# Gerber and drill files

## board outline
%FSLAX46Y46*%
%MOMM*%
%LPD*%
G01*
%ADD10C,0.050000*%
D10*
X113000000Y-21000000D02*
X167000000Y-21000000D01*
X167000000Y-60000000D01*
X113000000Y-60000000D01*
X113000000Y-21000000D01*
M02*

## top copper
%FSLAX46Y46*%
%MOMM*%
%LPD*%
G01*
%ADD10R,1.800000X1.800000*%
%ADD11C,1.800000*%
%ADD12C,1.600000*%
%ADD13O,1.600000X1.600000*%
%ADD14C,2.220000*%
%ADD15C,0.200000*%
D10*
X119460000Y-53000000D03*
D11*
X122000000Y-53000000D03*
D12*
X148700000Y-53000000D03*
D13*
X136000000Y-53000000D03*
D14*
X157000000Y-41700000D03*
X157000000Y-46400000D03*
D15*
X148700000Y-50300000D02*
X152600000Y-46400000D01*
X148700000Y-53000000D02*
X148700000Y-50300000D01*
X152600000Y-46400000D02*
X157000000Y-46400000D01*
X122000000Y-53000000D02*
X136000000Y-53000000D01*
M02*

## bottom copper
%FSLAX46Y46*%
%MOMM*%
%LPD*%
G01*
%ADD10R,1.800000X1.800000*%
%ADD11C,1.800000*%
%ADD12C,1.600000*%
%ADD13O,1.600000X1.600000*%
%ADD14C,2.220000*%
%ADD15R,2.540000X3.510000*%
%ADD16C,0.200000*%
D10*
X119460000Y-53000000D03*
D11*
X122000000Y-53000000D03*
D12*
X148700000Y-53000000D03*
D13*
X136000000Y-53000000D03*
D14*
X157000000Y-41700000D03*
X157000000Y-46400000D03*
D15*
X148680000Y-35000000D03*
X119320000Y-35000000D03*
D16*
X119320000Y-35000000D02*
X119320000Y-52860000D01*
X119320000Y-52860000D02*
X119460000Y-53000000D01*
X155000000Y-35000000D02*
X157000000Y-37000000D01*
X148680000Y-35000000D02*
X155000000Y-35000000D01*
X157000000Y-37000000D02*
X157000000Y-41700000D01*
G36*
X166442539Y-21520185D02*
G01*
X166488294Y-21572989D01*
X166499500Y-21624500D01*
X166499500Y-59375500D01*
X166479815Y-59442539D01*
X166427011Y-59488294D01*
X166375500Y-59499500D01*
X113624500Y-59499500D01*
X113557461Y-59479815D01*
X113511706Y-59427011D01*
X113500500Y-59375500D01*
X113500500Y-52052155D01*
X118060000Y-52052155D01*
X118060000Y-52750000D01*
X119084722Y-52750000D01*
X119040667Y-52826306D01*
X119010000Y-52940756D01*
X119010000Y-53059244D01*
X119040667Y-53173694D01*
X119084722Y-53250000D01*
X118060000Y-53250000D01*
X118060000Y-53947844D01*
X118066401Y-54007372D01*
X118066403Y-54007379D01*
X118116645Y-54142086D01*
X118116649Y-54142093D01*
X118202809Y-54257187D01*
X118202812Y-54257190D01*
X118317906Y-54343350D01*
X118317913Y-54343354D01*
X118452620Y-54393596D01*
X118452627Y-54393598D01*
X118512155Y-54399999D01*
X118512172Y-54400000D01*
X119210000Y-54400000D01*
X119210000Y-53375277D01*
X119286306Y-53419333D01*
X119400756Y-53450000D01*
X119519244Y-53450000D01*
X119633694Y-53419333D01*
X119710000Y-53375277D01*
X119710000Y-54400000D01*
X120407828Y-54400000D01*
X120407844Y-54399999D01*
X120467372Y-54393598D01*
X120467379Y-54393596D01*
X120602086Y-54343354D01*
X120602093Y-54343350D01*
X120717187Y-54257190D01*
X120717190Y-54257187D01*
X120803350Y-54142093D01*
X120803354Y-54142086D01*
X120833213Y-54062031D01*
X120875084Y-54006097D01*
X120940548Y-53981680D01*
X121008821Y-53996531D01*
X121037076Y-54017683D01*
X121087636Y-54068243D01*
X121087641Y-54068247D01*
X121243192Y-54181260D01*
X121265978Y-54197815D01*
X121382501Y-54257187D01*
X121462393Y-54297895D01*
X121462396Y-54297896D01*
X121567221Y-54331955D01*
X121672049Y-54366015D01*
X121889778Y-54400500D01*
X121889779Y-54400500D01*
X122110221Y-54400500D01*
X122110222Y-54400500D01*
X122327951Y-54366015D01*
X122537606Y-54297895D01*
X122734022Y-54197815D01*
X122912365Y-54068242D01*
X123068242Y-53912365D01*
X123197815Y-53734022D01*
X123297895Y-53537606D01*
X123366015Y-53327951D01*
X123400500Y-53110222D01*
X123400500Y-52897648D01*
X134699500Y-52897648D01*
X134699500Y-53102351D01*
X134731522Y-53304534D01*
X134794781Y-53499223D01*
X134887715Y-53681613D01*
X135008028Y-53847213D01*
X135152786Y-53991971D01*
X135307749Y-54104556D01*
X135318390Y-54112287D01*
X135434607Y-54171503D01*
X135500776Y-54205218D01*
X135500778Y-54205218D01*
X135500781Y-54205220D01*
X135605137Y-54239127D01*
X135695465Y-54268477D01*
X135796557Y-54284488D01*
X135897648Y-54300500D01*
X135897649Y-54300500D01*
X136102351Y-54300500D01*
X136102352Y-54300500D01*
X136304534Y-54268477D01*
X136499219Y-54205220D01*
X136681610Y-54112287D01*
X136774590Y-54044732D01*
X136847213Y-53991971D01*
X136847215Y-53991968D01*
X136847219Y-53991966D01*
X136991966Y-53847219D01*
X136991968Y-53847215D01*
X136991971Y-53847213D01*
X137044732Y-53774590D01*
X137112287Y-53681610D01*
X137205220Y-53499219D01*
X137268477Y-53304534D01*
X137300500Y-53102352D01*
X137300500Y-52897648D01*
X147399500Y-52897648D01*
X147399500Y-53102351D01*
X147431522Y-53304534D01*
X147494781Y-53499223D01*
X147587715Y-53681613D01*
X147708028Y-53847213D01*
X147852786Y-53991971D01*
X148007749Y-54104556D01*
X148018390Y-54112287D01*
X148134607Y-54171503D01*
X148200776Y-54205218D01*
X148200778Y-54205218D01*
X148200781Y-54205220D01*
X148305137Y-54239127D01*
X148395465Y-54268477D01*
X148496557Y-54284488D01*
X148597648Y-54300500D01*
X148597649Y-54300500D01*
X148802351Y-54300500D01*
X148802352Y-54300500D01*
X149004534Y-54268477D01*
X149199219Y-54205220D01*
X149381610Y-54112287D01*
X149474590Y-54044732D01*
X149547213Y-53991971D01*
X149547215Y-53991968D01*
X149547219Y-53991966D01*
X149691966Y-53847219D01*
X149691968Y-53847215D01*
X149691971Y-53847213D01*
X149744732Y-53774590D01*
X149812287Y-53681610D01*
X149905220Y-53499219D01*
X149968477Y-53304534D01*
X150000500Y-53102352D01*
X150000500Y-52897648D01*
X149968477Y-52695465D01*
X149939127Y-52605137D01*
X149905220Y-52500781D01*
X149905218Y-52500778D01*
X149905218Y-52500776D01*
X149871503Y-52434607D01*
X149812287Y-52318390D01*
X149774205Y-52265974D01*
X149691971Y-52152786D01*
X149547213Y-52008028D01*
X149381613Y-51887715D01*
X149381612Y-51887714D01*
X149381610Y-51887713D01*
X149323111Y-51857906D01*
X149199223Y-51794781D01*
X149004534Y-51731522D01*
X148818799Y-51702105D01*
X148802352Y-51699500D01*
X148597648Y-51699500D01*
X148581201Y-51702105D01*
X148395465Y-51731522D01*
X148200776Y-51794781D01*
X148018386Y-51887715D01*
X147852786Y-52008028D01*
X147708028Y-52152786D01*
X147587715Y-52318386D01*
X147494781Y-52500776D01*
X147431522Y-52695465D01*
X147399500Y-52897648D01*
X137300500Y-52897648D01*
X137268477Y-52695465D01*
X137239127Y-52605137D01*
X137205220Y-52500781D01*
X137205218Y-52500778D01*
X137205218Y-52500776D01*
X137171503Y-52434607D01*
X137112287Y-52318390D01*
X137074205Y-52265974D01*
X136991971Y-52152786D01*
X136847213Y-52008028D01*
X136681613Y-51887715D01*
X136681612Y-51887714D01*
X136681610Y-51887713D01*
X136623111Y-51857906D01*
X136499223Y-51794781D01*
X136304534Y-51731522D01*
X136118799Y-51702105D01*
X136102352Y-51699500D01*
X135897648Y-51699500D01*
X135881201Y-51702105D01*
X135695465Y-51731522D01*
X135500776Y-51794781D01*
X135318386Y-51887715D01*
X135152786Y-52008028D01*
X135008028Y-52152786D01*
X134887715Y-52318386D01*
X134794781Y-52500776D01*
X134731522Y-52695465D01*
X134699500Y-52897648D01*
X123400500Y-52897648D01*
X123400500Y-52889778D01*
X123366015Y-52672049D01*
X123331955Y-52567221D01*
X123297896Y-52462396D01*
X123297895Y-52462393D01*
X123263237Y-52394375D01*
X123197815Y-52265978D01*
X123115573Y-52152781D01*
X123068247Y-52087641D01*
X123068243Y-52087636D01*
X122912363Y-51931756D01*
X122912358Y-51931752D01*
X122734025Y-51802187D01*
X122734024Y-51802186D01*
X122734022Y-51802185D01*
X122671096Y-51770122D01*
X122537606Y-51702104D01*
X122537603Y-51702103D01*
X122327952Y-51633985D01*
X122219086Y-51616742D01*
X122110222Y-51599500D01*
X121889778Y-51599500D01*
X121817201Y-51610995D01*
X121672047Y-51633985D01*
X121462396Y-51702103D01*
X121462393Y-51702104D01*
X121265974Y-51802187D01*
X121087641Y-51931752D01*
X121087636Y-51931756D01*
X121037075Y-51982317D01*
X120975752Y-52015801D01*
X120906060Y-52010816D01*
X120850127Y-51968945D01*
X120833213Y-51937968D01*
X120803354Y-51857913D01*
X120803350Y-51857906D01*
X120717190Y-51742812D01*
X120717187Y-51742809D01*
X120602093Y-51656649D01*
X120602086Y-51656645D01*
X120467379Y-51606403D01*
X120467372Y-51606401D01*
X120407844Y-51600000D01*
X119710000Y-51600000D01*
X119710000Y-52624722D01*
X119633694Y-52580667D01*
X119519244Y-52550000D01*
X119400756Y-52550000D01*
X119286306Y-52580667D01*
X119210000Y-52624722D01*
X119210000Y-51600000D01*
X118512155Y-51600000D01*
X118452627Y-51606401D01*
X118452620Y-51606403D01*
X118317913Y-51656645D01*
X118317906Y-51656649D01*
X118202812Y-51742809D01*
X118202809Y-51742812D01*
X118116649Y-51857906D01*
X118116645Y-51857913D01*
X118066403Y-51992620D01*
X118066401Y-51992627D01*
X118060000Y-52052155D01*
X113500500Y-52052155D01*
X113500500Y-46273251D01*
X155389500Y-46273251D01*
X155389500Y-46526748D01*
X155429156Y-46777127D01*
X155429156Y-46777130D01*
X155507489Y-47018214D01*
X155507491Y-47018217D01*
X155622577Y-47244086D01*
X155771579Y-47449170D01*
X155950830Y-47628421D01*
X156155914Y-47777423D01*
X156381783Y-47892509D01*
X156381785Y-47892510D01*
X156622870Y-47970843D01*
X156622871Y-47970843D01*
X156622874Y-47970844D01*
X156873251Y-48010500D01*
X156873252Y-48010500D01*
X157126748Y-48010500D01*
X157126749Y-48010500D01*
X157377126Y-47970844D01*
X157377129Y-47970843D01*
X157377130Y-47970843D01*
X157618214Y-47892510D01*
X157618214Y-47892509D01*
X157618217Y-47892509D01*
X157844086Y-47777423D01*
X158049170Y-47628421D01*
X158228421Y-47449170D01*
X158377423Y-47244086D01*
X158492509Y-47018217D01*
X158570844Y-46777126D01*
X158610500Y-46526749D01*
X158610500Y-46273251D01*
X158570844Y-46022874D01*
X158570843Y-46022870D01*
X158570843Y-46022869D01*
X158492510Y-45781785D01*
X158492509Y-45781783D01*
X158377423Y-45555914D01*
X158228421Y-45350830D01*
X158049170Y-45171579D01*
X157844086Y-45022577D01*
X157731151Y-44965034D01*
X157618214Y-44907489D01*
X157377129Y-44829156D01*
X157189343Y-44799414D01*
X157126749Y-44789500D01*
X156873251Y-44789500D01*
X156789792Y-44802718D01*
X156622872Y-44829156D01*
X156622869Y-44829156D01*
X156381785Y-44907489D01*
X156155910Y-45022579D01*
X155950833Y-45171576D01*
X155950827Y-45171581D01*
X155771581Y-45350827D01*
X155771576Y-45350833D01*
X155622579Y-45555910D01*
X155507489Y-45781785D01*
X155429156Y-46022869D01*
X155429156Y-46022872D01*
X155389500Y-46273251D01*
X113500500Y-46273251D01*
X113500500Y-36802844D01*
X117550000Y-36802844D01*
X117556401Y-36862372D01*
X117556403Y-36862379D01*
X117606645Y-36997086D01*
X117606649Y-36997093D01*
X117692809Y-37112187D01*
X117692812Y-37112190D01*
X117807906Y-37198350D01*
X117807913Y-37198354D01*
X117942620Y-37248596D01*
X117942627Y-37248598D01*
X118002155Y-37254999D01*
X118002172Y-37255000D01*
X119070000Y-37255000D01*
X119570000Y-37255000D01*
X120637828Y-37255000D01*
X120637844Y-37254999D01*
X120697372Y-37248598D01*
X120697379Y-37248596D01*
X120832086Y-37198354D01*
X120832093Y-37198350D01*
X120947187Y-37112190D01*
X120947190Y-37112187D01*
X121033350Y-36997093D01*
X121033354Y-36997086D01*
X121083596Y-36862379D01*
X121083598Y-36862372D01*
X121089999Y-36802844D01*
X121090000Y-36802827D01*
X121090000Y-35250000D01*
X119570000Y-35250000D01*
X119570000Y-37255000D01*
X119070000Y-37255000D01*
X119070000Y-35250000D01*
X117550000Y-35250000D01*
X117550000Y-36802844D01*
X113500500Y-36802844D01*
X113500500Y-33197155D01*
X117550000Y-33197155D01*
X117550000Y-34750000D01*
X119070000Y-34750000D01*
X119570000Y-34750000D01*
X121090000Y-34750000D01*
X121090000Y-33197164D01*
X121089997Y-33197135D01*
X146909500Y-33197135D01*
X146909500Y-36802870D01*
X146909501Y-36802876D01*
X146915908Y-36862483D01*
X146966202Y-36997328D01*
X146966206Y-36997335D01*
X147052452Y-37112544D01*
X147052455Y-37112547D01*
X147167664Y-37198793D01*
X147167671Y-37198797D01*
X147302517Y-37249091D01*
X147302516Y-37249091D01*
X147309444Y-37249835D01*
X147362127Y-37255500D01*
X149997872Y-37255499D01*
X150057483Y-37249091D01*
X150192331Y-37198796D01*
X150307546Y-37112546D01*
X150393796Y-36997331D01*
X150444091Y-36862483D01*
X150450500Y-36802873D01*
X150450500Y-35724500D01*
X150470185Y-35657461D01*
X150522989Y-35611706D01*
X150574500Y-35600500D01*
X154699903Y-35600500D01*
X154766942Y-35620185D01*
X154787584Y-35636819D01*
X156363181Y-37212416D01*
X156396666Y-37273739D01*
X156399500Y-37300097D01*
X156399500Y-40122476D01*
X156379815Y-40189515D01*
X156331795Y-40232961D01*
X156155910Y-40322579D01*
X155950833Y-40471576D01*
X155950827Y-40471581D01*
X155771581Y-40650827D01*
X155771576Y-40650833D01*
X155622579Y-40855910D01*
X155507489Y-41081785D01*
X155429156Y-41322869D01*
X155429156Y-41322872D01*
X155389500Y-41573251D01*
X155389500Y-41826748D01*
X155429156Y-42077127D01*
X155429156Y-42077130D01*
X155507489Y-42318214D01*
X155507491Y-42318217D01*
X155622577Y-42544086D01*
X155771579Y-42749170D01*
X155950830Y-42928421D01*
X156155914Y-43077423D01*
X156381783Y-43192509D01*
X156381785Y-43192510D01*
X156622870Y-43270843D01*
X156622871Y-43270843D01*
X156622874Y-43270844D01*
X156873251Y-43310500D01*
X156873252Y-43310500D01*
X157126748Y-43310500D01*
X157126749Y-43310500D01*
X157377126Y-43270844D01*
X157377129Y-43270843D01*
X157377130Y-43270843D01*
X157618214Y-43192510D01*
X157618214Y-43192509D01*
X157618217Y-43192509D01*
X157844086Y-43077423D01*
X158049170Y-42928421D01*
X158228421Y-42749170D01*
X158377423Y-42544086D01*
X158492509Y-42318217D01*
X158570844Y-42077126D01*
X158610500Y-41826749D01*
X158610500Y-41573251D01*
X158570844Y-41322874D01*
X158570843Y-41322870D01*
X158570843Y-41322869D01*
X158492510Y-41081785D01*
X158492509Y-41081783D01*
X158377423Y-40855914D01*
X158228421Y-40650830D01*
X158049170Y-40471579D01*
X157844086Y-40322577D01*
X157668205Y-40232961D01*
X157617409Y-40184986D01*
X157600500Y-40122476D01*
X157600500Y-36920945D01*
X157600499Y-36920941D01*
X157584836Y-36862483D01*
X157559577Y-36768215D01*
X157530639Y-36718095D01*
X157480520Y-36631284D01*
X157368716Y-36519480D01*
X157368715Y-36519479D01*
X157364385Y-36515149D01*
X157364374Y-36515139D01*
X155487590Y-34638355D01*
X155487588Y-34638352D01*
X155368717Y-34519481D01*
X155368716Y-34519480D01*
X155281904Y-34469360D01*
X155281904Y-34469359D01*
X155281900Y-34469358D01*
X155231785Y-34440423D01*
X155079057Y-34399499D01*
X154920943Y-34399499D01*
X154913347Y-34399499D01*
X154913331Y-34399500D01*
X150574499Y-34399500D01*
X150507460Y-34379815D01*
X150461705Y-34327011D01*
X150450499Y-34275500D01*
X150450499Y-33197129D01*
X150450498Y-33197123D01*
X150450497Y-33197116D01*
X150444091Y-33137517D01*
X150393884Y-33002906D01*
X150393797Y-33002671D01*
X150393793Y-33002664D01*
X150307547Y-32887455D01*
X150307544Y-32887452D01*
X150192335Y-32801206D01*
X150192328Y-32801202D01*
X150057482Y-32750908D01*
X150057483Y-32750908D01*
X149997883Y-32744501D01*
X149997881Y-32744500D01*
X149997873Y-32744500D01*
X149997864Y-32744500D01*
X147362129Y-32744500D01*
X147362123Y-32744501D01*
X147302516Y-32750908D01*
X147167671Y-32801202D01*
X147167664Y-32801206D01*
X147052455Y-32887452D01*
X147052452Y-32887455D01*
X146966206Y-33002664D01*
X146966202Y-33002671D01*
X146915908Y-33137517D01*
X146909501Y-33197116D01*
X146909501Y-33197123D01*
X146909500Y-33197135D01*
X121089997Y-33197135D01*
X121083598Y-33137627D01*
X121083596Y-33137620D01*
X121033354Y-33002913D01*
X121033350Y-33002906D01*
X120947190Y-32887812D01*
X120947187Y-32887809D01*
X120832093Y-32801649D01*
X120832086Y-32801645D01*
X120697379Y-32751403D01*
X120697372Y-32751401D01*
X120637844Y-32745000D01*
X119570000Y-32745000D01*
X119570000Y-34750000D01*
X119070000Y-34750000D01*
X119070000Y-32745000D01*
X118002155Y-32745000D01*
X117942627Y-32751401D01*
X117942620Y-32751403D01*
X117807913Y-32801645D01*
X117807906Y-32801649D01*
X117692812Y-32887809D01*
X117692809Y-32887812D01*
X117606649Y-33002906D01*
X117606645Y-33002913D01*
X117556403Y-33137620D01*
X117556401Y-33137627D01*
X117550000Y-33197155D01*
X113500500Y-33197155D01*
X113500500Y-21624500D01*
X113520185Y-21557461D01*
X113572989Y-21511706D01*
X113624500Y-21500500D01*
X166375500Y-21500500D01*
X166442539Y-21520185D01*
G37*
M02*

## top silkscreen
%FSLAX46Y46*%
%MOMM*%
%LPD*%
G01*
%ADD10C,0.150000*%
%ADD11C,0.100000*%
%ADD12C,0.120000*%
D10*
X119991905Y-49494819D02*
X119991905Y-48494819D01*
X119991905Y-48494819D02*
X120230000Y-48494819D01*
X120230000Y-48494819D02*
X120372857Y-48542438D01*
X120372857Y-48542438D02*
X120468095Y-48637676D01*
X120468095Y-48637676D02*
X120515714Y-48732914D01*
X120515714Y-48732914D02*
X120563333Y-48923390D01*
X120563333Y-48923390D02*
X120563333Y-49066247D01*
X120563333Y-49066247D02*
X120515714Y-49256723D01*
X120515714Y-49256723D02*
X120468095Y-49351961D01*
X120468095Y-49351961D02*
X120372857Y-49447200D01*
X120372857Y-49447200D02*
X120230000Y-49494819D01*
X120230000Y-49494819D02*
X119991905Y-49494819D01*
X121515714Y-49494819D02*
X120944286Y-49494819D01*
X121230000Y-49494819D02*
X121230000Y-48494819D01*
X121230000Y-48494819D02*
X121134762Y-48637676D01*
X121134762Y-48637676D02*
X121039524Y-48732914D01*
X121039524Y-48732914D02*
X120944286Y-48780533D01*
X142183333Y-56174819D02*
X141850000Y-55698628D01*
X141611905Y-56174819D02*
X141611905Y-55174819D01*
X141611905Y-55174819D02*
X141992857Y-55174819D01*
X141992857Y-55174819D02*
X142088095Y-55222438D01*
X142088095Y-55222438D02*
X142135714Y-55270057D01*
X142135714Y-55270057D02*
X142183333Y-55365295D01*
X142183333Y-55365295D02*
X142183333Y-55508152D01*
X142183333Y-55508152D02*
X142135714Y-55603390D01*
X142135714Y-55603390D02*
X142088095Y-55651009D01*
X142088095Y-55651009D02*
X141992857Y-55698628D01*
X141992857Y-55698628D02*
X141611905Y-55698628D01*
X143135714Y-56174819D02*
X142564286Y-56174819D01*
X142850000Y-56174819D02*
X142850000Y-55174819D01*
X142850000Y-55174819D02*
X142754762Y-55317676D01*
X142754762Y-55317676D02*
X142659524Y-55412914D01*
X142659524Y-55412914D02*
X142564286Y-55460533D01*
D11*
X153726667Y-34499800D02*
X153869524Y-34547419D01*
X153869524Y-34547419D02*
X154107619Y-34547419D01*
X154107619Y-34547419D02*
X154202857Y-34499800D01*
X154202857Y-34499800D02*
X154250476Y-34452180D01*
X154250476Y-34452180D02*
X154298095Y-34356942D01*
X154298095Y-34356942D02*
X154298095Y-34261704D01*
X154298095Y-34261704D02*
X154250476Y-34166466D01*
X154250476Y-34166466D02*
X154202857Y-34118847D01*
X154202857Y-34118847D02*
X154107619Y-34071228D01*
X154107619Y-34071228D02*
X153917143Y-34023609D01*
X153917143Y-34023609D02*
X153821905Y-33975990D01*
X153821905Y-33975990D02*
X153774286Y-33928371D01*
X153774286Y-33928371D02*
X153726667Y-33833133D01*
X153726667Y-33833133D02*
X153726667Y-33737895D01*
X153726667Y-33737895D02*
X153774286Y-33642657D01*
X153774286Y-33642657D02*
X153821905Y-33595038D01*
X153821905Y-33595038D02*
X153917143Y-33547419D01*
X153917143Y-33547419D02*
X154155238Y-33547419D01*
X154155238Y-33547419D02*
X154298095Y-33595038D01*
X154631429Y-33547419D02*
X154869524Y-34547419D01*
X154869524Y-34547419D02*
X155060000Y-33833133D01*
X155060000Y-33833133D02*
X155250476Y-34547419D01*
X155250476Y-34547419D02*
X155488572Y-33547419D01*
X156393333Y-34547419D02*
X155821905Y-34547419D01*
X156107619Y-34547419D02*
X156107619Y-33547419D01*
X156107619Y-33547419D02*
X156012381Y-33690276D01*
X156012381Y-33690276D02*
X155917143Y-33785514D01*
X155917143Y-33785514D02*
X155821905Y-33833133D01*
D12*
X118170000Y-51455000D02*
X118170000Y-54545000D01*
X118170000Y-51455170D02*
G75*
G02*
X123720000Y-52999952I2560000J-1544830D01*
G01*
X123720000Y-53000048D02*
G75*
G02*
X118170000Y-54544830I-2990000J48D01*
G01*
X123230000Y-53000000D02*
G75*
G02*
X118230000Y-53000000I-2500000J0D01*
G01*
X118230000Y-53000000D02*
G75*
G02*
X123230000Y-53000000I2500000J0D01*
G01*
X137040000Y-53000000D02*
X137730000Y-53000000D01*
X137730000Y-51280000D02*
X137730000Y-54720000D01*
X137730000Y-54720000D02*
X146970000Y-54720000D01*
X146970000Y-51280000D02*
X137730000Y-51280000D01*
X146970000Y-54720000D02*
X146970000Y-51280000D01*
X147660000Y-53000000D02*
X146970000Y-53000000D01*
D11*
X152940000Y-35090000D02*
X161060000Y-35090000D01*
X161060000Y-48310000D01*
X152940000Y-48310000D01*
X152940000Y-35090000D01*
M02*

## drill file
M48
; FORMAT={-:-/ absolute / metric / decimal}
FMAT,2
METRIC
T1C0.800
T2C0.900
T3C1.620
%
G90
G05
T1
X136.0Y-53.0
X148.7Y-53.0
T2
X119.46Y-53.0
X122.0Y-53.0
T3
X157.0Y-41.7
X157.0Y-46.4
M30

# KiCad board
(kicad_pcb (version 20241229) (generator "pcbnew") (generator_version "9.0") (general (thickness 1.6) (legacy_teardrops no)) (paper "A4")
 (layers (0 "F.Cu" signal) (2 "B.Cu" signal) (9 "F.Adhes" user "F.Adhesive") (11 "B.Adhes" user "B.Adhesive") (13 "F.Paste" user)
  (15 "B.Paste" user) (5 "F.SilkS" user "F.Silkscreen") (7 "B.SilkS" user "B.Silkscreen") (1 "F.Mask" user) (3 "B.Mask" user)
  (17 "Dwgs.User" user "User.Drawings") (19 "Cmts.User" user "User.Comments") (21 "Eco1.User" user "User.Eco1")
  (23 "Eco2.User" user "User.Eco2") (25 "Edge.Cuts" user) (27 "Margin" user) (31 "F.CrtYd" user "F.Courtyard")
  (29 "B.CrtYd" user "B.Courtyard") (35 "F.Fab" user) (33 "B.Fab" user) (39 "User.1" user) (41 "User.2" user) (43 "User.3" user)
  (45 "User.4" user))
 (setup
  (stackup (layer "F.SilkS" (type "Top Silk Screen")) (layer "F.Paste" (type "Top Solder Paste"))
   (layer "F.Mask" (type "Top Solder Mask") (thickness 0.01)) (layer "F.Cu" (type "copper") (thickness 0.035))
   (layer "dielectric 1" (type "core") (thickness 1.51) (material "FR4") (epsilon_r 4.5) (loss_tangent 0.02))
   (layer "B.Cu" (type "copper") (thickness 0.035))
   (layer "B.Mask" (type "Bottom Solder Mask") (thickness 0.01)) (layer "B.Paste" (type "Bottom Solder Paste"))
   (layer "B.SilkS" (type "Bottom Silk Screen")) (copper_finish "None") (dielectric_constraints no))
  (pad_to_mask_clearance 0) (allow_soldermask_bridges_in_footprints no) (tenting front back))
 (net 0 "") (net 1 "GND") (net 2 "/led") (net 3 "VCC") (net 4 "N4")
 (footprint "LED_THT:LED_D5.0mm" (layer "F.Cu") (at 119.46 53)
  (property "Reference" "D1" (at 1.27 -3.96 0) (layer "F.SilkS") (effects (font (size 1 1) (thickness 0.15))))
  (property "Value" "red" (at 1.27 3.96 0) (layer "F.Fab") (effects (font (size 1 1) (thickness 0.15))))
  (fp_line (start -1.29 -1.545) (end -1.29 1.545) (stroke (width 0.12) (type solid)) (layer "F.SilkS"))
  (fp_arc (start -1.29 -1.54483) (mid 2.071756 -2.880501) (end 4.26 -0.000048) (stroke (width 0.12) (type solid)) (layer "F.SilkS"))
  (fp_arc (start 4.26 0.000048) (mid 2.071756 2.880501) (end -1.29 1.54483) (stroke (width 0.12) (type solid)) (layer "F.SilkS"))
  (fp_circle (center 1.27 0) (end 3.77 0) (stroke (width 0.12) (type solid)) (fill no) (layer "F.SilkS"))
  (pad "1" thru_hole rect (at 0 0) (size 1.8 1.8) (drill 0.9) (layers "*.Cu" "*.Mask") (remove_unused_layers no) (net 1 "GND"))
  (pad "2" thru_hole circle (at 2.54 0) (size 1.8 1.8) (drill 0.9) (layers "*.Cu" "*.Mask") (remove_unused_layers no) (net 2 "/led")))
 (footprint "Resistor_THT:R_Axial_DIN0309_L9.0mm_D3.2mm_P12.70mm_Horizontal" (layer "F.Cu") (at 148.7 53 180)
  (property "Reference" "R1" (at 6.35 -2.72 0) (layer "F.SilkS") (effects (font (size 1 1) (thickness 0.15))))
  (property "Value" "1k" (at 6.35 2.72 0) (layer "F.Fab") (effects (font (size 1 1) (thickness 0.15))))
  (fp_line (start 11.66 0) (end 10.97 0) (stroke (width 0.12) (type solid)) (layer "F.SilkS"))
  (fp_line (start 10.97 1.72) (end 10.97 -1.72) (stroke (width 0.12) (type solid)) (layer "F.SilkS"))
  (fp_line (start 10.97 -1.72) (end 1.73 -1.72) (stroke (width 0.12) (type solid)) (layer "F.SilkS"))
  (fp_line (start 1.73 1.72) (end 10.97 1.72) (stroke (width 0.12) (type solid)) (layer "F.SilkS"))
  (fp_line (start 1.73 -1.72) (end 1.73 1.72) (stroke (width 0.12) (type solid)) (layer "F.SilkS"))
  (fp_line (start 1.04 0) (end 1.73 0) (stroke (width 0.12) (type solid)) (layer "F.SilkS"))
  (pad "1" thru_hole circle (at 0 0 180) (size 1.6 1.6) (drill 0.8) (layers "*.Cu" "*.Mask") (remove_unused_layers no) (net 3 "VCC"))
  (pad "2" thru_hole oval (at 12.7 0 180) (size 1.6 1.6) (drill 0.8) (layers "*.Cu" "*.Mask") (remove_unused_layers no) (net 2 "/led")))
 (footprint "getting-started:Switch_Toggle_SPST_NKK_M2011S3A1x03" (layer "F.Cu") (at 157 37)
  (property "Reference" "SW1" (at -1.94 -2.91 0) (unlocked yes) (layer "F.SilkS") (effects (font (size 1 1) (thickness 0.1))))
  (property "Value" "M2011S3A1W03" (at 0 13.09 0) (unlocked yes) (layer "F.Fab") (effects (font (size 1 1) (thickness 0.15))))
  (fp_rect (start -4.06 -1.91) (end 4.06 11.31) (stroke (width 0.1) (type default)) (fill no) (layer "F.SilkS"))
  (pad "2" thru_hole circle (at 0 4.7) (size 2.22 2.22) (drill 1.62) (layers "*.Cu" "*.Mask") (remove_unused_layers no) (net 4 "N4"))
  (pad "3" thru_hole circle (at 0 9.4) (size 2.22 2.22) (drill 1.62) (layers "*.Cu" "*.Mask") (remove_unused_layers no) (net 3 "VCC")))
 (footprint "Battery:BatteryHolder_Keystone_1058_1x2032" (layer "B.Cu") (at 134 35 180)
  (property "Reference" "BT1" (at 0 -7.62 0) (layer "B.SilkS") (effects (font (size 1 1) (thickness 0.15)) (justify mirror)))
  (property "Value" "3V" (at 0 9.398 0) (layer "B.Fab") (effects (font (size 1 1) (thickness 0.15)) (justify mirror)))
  (pad "1" smd rect (at -14.68 0 180) (size 2.54 3.51) (layers "B.Cu" "B.Mask" "B.Paste") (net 4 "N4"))
  (pad "2" smd rect (at 14.68 0 180) (size 2.54 3.51) (layers "B.Cu" "B.Mask" "B.Paste") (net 1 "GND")))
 (gr_rect (start 113 21) (end 167 60) (stroke (width 0.05) (type default)) (fill no) (layer "Edge.Cuts"))
 (segment (start 119.32 35) (end 119.32 52.86) (width 0.2) (layer "B.Cu") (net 1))
 (segment (start 119.32 52.86) (end 119.46 53) (width 0.2) (layer "B.Cu") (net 1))
 (segment (start 148.7 50.3) (end 152.6 46.4) (width 0.2) (layer "F.Cu") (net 3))
 (segment (start 148.7 53) (end 148.7 50.3) (width 0.2) (layer "F.Cu") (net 3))
 (segment (start 152.6 46.4) (end 157 46.4) (width 0.2) (layer "F.Cu") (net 3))
 (segment (start 122 53) (end 136 53) (width 0.2) (layer "F.Cu") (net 2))
 (segment (start 155 35) (end 157 37) (width 0.2) (layer "B.Cu") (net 4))
 (segment (start 148.68 35) (end 155 35) (width 0.2) (layer "B.Cu") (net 4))
 (segment (start 157 37) (end 157 41.7) (width 0.2) (layer "B.Cu") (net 4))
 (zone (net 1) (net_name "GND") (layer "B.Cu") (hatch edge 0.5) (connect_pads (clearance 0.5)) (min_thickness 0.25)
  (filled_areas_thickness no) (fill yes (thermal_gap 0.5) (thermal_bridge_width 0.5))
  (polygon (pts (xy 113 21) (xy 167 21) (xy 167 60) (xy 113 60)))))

